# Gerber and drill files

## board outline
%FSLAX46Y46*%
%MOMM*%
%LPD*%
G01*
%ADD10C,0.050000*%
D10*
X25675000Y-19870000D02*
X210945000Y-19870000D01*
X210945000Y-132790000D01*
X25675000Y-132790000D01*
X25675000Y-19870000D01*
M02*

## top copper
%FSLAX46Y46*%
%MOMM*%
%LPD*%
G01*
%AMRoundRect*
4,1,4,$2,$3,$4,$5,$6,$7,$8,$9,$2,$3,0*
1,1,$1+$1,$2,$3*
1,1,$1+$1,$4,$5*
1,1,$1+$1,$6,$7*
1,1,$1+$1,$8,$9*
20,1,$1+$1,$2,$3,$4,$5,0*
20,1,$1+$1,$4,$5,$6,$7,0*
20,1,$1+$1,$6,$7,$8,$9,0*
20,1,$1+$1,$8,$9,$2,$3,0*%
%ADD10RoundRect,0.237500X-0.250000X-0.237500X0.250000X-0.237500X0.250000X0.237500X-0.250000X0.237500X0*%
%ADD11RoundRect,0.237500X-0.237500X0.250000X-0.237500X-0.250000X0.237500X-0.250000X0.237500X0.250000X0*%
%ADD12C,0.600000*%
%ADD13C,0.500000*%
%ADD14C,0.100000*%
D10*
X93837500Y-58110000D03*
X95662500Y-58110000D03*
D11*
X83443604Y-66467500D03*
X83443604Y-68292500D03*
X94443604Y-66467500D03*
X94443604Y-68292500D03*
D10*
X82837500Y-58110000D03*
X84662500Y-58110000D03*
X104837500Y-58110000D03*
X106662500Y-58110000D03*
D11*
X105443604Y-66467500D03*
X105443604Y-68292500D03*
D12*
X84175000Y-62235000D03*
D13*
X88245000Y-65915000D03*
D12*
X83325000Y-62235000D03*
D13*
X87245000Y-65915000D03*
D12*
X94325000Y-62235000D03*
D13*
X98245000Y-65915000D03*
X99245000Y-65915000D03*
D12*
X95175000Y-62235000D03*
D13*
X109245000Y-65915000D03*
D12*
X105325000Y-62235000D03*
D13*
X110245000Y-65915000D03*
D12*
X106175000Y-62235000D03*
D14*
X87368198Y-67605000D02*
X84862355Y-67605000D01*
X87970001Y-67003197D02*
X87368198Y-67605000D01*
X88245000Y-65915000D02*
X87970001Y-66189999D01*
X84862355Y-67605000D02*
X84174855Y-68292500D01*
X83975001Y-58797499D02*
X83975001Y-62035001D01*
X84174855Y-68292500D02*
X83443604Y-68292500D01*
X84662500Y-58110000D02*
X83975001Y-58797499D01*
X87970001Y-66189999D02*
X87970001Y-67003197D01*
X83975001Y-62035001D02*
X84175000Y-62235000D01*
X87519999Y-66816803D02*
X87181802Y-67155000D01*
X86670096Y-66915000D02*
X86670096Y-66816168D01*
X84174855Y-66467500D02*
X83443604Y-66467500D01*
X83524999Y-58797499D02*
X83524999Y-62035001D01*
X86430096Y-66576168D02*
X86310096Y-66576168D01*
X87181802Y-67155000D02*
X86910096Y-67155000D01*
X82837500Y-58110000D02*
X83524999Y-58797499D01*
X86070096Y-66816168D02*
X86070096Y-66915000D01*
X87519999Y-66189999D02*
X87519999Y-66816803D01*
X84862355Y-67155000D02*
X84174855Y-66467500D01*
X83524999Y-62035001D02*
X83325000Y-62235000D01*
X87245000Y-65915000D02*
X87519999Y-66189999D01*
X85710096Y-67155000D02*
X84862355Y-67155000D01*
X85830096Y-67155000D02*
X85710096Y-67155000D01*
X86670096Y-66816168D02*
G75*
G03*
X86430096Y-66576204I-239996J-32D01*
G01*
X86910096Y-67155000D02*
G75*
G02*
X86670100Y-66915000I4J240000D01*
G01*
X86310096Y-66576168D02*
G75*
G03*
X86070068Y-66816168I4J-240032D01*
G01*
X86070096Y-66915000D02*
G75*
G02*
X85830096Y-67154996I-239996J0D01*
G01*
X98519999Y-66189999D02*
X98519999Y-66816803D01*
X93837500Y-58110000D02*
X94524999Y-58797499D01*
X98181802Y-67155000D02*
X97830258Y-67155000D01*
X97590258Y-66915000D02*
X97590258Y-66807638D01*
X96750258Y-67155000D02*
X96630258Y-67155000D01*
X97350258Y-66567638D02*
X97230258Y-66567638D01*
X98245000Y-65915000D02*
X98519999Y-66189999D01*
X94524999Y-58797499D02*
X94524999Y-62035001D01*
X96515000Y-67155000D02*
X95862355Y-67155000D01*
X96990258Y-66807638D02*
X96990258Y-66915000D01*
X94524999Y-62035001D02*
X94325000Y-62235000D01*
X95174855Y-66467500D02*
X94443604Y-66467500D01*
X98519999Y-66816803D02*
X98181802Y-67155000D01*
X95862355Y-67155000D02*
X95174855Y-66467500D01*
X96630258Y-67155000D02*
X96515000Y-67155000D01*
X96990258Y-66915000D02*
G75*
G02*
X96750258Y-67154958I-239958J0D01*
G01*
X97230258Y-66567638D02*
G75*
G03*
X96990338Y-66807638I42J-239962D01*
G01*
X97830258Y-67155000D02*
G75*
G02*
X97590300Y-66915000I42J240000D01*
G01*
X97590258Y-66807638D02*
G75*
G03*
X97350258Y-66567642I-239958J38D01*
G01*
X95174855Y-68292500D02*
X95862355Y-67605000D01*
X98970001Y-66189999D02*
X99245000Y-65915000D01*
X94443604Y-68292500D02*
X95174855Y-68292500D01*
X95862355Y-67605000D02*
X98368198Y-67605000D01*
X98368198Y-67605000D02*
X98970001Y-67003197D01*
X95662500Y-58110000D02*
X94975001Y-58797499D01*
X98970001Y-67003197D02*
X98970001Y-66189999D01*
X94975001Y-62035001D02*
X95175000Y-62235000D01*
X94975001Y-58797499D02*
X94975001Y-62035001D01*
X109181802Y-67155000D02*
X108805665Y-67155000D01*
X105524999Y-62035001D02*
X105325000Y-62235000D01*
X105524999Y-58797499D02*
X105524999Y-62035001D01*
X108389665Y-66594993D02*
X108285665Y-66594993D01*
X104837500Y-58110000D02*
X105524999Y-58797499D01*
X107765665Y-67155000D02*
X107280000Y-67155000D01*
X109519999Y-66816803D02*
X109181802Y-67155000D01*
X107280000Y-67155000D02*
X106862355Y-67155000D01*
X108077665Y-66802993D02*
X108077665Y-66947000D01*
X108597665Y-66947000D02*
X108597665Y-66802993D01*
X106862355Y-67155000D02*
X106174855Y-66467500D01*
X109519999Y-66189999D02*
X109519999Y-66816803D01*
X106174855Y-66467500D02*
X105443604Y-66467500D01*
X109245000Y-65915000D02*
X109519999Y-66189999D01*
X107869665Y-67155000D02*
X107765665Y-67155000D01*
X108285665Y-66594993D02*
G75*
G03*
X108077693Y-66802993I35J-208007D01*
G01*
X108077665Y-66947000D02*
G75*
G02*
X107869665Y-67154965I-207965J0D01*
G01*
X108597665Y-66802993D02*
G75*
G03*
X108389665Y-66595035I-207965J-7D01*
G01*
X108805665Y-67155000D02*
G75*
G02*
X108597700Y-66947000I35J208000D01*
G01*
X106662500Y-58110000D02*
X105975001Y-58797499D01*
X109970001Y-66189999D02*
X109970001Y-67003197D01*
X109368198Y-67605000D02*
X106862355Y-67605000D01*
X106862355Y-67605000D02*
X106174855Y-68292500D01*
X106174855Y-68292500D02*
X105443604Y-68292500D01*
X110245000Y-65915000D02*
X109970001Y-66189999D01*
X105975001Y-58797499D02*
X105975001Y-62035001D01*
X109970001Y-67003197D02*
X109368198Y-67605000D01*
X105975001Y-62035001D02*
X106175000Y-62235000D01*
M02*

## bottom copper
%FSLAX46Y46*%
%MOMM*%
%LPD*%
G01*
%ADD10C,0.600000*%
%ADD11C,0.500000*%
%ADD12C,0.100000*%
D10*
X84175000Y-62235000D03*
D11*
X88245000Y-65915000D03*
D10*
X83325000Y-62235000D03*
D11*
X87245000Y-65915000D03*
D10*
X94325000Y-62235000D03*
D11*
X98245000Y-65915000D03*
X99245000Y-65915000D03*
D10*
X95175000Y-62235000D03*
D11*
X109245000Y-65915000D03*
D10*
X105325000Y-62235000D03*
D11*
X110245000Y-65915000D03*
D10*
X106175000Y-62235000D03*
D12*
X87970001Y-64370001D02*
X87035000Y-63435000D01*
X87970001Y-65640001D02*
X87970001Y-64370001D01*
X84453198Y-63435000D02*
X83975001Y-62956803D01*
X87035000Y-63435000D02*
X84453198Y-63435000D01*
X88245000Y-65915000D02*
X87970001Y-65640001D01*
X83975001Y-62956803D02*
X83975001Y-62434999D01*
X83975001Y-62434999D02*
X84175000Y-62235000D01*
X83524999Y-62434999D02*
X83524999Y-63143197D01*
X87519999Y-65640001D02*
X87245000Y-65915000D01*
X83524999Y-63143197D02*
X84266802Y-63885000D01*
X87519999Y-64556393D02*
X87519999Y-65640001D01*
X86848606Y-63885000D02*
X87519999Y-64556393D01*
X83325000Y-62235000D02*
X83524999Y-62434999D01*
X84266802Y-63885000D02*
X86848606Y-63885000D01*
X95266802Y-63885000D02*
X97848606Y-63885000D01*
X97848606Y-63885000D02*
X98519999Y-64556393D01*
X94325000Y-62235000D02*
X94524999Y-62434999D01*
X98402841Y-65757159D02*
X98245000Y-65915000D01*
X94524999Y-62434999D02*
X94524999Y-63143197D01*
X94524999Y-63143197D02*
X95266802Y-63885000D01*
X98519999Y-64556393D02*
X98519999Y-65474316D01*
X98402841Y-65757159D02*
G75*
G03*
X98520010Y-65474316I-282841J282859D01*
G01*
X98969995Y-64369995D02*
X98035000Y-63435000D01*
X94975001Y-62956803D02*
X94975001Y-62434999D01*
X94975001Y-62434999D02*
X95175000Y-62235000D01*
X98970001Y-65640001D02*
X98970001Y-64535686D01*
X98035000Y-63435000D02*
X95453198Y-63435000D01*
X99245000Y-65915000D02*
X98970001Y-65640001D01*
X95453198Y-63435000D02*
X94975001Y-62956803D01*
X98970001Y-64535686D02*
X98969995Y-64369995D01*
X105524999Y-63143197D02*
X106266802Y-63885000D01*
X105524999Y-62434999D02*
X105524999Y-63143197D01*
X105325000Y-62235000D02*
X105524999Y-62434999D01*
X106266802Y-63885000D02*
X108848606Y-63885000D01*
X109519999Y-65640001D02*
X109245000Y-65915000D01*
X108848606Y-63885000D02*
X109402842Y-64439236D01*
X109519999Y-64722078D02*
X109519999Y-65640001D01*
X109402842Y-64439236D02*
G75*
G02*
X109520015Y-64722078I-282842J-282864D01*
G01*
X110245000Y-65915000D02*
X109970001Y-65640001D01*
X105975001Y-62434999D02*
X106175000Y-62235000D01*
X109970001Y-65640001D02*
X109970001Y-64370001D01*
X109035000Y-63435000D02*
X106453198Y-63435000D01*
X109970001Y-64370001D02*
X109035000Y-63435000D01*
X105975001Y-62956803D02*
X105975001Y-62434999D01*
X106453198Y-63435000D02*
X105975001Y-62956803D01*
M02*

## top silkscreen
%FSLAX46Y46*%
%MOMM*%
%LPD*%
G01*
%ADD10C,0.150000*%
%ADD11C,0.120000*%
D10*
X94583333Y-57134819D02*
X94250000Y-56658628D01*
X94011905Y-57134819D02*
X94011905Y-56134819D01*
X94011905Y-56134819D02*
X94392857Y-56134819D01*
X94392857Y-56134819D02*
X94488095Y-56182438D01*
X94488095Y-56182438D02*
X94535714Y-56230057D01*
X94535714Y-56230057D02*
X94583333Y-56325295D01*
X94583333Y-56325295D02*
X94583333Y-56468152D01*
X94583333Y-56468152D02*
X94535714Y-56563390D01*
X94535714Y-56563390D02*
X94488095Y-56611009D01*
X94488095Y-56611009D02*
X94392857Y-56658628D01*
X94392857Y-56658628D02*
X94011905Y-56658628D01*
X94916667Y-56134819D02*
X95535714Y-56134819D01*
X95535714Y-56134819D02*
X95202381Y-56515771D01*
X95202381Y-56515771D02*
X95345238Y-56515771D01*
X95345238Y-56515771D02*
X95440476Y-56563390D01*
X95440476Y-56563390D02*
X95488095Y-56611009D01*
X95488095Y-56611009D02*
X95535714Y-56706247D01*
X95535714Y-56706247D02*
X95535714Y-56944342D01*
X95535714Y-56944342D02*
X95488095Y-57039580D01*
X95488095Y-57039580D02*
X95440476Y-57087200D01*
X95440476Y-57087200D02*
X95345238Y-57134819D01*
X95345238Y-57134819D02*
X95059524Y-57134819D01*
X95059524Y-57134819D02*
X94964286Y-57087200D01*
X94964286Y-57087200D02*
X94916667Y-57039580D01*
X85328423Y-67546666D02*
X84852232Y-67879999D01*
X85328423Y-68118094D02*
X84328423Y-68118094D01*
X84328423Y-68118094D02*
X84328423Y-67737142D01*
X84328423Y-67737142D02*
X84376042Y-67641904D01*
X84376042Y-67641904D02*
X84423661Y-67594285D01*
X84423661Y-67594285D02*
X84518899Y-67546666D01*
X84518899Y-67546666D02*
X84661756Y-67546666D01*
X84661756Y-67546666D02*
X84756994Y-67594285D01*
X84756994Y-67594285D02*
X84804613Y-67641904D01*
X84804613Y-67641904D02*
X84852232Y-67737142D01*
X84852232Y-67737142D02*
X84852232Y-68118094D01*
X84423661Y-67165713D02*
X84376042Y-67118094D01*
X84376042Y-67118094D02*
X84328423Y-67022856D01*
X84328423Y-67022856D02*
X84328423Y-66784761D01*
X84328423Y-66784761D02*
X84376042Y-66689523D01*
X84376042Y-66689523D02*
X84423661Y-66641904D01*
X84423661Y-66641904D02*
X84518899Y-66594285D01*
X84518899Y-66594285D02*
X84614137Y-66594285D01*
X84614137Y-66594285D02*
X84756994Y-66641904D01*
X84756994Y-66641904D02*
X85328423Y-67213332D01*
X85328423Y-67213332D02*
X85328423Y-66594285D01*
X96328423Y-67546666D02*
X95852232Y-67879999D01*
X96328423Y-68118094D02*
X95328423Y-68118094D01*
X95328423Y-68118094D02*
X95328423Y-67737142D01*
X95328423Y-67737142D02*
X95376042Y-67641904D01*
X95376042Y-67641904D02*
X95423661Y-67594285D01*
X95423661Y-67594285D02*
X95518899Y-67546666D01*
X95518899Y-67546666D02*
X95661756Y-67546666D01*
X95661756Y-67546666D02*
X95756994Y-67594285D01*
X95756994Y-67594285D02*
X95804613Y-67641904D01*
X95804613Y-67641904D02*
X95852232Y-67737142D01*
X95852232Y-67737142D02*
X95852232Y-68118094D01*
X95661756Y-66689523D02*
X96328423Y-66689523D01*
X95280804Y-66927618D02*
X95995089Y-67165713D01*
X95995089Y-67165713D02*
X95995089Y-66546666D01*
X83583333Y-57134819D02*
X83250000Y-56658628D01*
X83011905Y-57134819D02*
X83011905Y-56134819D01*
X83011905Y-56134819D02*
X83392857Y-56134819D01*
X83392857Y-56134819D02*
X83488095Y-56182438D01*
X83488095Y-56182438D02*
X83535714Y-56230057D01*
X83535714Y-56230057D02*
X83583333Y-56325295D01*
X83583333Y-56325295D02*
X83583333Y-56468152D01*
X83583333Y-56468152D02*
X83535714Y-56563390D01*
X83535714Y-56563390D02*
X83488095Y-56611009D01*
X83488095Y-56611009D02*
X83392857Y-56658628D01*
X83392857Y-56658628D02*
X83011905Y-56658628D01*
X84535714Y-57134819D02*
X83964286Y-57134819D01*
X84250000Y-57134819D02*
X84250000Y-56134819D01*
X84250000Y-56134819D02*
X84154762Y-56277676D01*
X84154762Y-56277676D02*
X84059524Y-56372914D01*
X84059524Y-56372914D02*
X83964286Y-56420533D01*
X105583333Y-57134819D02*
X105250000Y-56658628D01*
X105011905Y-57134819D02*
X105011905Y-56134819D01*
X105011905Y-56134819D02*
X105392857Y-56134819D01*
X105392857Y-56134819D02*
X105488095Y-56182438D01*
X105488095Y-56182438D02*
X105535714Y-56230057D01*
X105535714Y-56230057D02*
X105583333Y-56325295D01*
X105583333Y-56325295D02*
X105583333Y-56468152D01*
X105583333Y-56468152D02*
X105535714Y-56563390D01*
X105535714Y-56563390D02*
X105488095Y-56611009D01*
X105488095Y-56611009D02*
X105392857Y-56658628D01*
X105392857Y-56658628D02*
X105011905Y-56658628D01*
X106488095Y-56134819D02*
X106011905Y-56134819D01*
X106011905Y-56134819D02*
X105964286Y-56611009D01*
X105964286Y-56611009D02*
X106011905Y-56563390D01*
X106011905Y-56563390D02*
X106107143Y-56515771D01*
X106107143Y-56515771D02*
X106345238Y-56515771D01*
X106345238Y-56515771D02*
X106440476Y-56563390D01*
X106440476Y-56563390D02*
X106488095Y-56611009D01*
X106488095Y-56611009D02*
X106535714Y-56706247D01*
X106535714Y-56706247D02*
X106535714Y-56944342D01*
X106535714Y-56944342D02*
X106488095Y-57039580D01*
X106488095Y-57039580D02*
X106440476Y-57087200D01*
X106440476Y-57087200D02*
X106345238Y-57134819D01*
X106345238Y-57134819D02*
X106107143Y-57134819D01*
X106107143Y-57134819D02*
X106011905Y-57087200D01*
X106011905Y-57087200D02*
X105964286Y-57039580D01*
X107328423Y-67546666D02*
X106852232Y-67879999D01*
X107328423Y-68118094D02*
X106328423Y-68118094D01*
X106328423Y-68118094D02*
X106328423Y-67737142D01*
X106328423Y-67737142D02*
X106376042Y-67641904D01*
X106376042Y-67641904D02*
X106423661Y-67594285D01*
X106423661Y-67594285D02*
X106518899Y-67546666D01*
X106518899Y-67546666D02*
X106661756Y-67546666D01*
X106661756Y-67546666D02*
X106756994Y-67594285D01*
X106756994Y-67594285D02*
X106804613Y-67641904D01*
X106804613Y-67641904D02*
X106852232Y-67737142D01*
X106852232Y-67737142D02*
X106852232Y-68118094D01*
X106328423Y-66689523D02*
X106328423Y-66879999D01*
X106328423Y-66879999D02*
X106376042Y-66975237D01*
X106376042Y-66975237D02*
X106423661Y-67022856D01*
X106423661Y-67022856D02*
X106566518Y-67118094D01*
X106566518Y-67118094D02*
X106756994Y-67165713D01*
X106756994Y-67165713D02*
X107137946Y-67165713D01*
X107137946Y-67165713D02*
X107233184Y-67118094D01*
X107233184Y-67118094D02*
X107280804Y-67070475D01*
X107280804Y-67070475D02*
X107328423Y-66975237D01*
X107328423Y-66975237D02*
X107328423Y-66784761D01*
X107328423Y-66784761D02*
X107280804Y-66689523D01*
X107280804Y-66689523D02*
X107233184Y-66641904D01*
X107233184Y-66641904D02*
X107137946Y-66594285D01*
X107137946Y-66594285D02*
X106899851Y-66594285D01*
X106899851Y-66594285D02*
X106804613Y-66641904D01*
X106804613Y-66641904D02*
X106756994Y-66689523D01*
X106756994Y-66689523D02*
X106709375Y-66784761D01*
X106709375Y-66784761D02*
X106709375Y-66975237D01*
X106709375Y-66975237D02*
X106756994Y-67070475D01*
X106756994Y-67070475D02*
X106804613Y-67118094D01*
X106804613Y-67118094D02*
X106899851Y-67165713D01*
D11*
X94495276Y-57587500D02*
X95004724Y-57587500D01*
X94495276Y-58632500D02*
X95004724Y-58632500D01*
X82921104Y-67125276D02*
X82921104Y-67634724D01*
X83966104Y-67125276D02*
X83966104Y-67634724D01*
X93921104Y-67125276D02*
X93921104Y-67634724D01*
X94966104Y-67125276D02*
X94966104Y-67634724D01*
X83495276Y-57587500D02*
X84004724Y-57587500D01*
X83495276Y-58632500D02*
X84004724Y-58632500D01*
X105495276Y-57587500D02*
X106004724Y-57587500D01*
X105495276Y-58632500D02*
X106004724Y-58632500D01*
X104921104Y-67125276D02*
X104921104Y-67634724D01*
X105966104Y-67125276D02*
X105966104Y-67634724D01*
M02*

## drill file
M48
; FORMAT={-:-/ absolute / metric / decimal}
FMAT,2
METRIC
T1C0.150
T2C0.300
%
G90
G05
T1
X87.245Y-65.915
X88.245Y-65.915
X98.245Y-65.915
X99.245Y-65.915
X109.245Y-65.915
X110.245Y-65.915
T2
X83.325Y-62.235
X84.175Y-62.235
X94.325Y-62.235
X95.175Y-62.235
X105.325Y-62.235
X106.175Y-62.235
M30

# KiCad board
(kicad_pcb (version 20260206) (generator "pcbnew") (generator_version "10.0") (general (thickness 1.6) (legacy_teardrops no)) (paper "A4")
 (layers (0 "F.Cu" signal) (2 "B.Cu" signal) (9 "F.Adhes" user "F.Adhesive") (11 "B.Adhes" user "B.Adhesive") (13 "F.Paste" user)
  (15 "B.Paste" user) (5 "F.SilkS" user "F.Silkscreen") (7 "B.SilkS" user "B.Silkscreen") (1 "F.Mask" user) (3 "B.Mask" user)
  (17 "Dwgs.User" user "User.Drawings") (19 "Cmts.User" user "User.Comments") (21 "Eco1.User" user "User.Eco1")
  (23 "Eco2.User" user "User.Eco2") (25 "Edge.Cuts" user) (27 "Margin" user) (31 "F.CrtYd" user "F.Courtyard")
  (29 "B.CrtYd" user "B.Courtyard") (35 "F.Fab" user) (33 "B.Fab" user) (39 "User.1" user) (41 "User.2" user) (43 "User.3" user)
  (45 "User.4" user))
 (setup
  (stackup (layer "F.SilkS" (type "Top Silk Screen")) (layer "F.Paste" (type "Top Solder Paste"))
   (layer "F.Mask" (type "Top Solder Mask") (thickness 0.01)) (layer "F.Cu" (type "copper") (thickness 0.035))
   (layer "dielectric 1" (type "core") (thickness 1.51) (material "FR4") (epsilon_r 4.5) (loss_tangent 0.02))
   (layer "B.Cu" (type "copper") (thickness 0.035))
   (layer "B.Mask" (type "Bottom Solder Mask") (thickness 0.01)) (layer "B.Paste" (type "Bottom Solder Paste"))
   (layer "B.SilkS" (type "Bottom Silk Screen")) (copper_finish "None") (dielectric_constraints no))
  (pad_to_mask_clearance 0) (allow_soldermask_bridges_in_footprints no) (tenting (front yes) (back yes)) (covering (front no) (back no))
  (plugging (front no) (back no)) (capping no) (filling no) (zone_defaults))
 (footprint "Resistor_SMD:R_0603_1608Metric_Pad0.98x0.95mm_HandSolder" (layer "F.Cu") (at 94.75 58.11)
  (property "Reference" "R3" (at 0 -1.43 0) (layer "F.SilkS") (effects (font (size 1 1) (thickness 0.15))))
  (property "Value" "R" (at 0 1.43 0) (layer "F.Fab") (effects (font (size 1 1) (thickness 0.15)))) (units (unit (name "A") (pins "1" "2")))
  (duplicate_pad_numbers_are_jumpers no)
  (fp_line (start -0.254724 -0.5225) (end 0.254724 -0.5225) (stroke (width 0.12) (type solid)) (layer "F.SilkS"))
  (fp_line (start -0.254724 0.5225) (end 0.254724 0.5225) (stroke (width 0.12) (type solid)) (layer "F.SilkS"))
  (pad "1" smd roundrect (at -0.9125 0) (size 0.975 0.95) (layers "F.Cu" "F.Mask" "F.Paste") (roundrect_rratio 0.25) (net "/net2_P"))
  (pad "2" smd roundrect (at 0.9125 0) (size 0.975 0.95) (layers "F.Cu" "F.Mask" "F.Paste") (roundrect_rratio 0.25) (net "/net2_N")))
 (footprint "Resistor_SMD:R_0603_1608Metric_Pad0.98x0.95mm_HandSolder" (layer "F.Cu") (at 83.443604 67.38 -90)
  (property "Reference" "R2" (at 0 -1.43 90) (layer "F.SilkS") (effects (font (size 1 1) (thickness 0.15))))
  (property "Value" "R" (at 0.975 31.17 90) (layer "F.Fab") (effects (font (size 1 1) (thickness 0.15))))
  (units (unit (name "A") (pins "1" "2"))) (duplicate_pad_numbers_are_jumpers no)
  (fp_line (start -0.254724 0.5225) (end 0.254724 0.5225) (stroke (width 0.12) (type solid)) (layer "F.SilkS"))
  (fp_line (start -0.254724 -0.5225) (end 0.254724 -0.5225) (stroke (width 0.12) (type solid)) (layer "F.SilkS"))
  (pad "1" smd roundrect (at -0.9125 0 270) (size 0.975 0.95) (layers "F.Cu" "F.Mask" "F.Paste") (roundrect_rratio 0.25) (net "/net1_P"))
  (pad "2" smd roundrect (at 0.9125 0 270) (size 0.975 0.95) (layers "F.Cu" "F.Mask" "F.Paste") (roundrect_rratio 0.25) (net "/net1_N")))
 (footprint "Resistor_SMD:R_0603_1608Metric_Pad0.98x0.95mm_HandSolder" (layer "F.Cu") (at 94.443604 67.38 -90)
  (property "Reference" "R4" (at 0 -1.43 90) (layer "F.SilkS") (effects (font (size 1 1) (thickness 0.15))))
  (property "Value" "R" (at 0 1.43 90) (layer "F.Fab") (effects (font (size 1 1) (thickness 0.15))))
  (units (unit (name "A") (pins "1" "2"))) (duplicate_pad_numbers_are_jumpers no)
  (fp_line (start -0.254724 0.5225) (end 0.254724 0.5225) (stroke (width 0.12) (type solid)) (layer "F.SilkS"))
  (fp_line (start -0.254724 -0.5225) (end 0.254724 -0.5225) (stroke (width 0.12) (type solid)) (layer "F.SilkS"))
  (pad "1" smd roundrect (at -0.9125 0 270) (size 0.975 0.95) (layers "F.Cu" "F.Mask" "F.Paste") (roundrect_rratio 0.25) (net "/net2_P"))
  (pad "2" smd roundrect (at 0.9125 0 270) (size 0.975 0.95) (layers "F.Cu" "F.Mask" "F.Paste") (roundrect_rratio 0.25) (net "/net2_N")))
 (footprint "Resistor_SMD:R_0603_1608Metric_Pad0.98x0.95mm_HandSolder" (layer "F.Cu") (at 83.75 58.11)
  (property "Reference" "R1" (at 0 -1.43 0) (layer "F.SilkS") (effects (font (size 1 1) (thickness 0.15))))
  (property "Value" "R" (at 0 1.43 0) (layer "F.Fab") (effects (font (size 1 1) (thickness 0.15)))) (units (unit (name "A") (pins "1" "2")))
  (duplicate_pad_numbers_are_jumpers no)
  (fp_line (start -0.254724 -0.5225) (end 0.254724 -0.5225) (stroke (width 0.12) (type solid)) (layer "F.SilkS"))
  (fp_line (start -0.254724 0.5225) (end 0.254724 0.5225) (stroke (width 0.12) (type solid)) (layer "F.SilkS"))
  (pad "1" smd roundrect (at -0.9125 0) (size 0.975 0.95) (layers "F.Cu" "F.Mask" "F.Paste") (roundrect_rratio 0.25) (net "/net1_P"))
  (pad "2" smd roundrect (at 0.9125 0) (size 0.975 0.95) (layers "F.Cu" "F.Mask" "F.Paste") (roundrect_rratio 0.25) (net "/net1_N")))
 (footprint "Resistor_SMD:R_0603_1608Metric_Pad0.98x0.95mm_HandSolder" (layer "F.Cu") (at 105.75 58.11)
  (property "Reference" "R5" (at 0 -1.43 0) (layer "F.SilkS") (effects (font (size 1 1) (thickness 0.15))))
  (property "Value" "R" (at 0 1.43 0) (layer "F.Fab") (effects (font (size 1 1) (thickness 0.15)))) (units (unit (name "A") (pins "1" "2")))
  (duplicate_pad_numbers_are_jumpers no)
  (fp_line (start -0.254724 -0.5225) (end 0.254724 -0.5225) (stroke (width 0.12) (type solid)) (layer "F.SilkS"))
  (fp_line (start -0.254724 0.5225) (end 0.254724 0.5225) (stroke (width 0.12) (type solid)) (layer "F.SilkS"))
  (pad "1" smd roundrect (at -0.9125 0) (size 0.975 0.95) (layers "F.Cu" "F.Mask" "F.Paste") (roundrect_rratio 0.25) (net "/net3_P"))
  (pad "2" smd roundrect (at 0.9125 0) (size 0.975 0.95) (layers "F.Cu" "F.Mask" "F.Paste") (roundrect_rratio 0.25) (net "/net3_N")))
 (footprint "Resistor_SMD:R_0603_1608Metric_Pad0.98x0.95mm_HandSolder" (layer "F.Cu") (at 105.443604 67.38 -90)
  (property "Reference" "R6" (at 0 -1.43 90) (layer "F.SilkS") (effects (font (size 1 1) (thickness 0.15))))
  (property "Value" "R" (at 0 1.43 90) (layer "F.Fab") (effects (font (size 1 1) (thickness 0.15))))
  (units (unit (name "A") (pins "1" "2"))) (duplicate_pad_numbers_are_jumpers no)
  (fp_line (start -0.254724 0.5225) (end 0.254724 0.5225) (stroke (width 0.12) (type solid)) (layer "F.SilkS"))
  (fp_line (start -0.254724 -0.5225) (end 0.254724 -0.5225) (stroke (width 0.12) (type solid)) (layer "F.SilkS"))
  (pad "1" smd roundrect (at -0.9125 0 270) (size 0.975 0.95) (layers "F.Cu" "F.Mask" "F.Paste") (roundrect_rratio 0.25) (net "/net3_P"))
  (pad "2" smd roundrect (at 0.9125 0 270) (size 0.975 0.95) (layers "F.Cu" "F.Mask" "F.Paste") (roundrect_rratio 0.25) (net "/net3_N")))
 (gr_rect (start 25.675 19.87) (end 210.945 132.79) (stroke (width 0.05) (type default)) (fill no) (layer "Edge.Cuts"))
 (segment (start 87.368198 67.605) (end 84.862355 67.605) (width 0.1) (layer "F.Cu") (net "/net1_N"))
 (segment (start 87.970001 67.003197) (end 87.368198 67.605) (width 0.1) (layer "F.Cu") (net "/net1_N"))
 (segment (start 88.245 65.915) (end 87.970001 66.189999) (width 0.1) (layer "F.Cu") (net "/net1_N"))
 (segment (start 84.862355 67.605) (end 84.174855 68.2925) (width 0.1) (layer "F.Cu") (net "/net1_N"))
 (segment (start 83.975001 58.797499) (end 83.975001 62.035001) (width 0.1) (layer "F.Cu") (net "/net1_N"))
 (segment (start 84.174855 68.2925) (end 83.443604 68.2925) (width 0.1) (layer "F.Cu") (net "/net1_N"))
 (segment (start 84.6625 58.11) (end 83.975001 58.797499) (width 0.1) (layer "F.Cu") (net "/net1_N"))
 (segment (start 87.970001 66.189999) (end 87.970001 67.003197) (width 0.1) (layer "F.Cu") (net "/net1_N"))
 (segment (start 83.975001 62.035001) (end 84.175 62.235) (width 0.1) (layer "F.Cu") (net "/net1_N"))
 (via (at 84.175 62.235) (size 0.6) (drill 0.3) (layers "F.Cu" "B.Cu") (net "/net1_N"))
 (via (at 88.245 65.915) (size 0.5) (drill 0.15) (layers "F.Cu" "B.Cu") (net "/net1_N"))
 (segment (start 87.970001 64.370001) (end 87.035 63.435) (width 0.1) (layer "B.Cu") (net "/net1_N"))
 (segment (start 87.970001 65.640001) (end 87.970001 64.370001) (width 0.1) (layer "B.Cu") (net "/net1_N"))
 (segment (start 84.453198 63.435) (end 83.975001 62.956803) (width 0.1) (layer "B.Cu") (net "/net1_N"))
 (segment (start 87.035 63.435) (end 84.453198 63.435) (width 0.1) (layer "B.Cu") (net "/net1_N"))
 (segment (start 88.245 65.915) (end 87.970001 65.640001) (width 0.1) (layer "B.Cu") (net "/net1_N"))
 (segment (start 83.975001 62.956803) (end 83.975001 62.434999) (width 0.1) (layer "B.Cu") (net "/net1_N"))
 (segment (start 83.975001 62.434999) (end 84.175 62.235) (width 0.1) (layer "B.Cu") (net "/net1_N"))
 (segment (start 87.519999 66.816803) (end 87.181802 67.155) (width 0.1) (layer "F.Cu") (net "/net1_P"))
 (segment (start 86.670096 66.915) (end 86.670096 66.816168) (width 0.1) (layer "F.Cu") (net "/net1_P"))
 (segment (start 84.174855 66.4675) (end 83.443604 66.4675) (width 0.1) (layer "F.Cu") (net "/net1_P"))
 (segment (start 83.524999 58.797499) (end 83.524999 62.035001) (width 0.1) (layer "F.Cu") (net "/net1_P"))
 (segment (start 86.430096 66.576168) (end 86.310096 66.576168) (width 0.1) (layer "F.Cu") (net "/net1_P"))
 (segment (start 87.181802 67.155) (end 86.910096 67.155) (width 0.1) (layer "F.Cu") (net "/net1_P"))
 (segment (start 82.8375 58.11) (end 83.524999 58.797499) (width 0.1) (layer "F.Cu") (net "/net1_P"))
 (segment (start 86.070096 66.816168) (end 86.070096 66.915) (width 0.1) (layer "F.Cu") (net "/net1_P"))
 (segment (start 87.519999 66.189999) (end 87.519999 66.816803) (width 0.1) (layer "F.Cu") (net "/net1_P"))
 (segment (start 84.862355 67.155) (end 84.174855 66.4675) (width 0.1) (layer "F.Cu") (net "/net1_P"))
 (segment (start 83.524999 62.035001) (end 83.325 62.235) (width 0.1) (layer "F.Cu") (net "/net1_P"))
 (segment (start 87.245 65.915) (end 87.519999 66.189999) (width 0.1) (layer "F.Cu") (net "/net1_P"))
 (segment (start 85.710096 67.155) (end 84.862355 67.155) (width 0.1) (layer "F.Cu") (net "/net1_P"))
 (segment (start 85.830096 67.155) (end 85.710096 67.155) (width 0.1) (layer "F.Cu") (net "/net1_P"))
 (via (at 83.325 62.235) (size 0.6) (drill 0.3) (layers "F.Cu" "B.Cu") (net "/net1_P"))
 (via (at 87.245 65.915) (size 0.5) (drill 0.15) (layers "F.Cu" "B.Cu") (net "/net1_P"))
 (arc (start 86.670096 66.816168) (mid 86.599802 66.646462) (end 86.430096 66.576168) (width 0.1) (layer "F.Cu") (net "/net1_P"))
 (arc (start 86.910096 67.155) (mid 86.74039 67.084706) (end 86.670096 66.915) (width 0.1) (layer "F.Cu") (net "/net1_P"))
 (arc (start 86.310096 66.576168) (mid 86.14039 66.646462) (end 86.070096 66.816168) (width 0.1) (layer "F.Cu") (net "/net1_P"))
 (arc (start 86.070096 66.915) (mid 85.999802 67.084706) (end 85.830096 67.155) (width 0.1) (layer "F.Cu") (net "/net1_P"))
 (segment (start 83.524999 62.434999) (end 83.524999 63.143197) (width 0.1) (layer "B.Cu") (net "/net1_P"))
 (segment (start 87.519999 65.640001) (end 87.245 65.915) (width 0.1) (layer "B.Cu") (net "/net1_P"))
 (segment (start 83.524999 63.143197) (end 84.266802 63.885) (width 0.1) (layer "B.Cu") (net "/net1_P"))
 (segment (start 87.519999 64.556393) (end 87.519999 65.640001) (width 0.1) (layer "B.Cu") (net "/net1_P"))
 (segment (start 86.848606 63.885) (end 87.519999 64.556393) (width 0.1) (layer "B.Cu") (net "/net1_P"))
 (segment (start 83.325 62.235) (end 83.524999 62.434999) (width 0.1) (layer "B.Cu") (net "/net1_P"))
 (segment (start 84.266802 63.885) (end 86.848606 63.885) (width 0.1) (layer "B.Cu") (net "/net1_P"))
 (segment (start 98.519999 66.189999) (end 98.519999 66.816803) (width 0.1) (layer "F.Cu") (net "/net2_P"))
 (segment (start 93.8375 58.11) (end 94.524999 58.797499) (width 0.1) (layer "F.Cu") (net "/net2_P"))
 (segment (start 98.181802 67.155) (end 97.830258 67.155) (width 0.1) (layer "F.Cu") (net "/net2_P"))
 (segment (start 97.590258 66.915) (end 97.590258 66.807638) (width 0.1) (layer "F.Cu") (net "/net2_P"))
 (segment (start 96.750258 67.155) (end 96.630258 67.155) (width 0.1) (layer "F.Cu") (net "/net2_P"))
 (segment (start 97.350258 66.567638) (end 97.230258 66.567638) (width 0.1) (layer "F.Cu") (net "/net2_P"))
 (segment (start 98.245 65.915) (end 98.519999 66.189999) (width 0.1) (layer "F.Cu") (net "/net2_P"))
 (segment (start 94.524999 58.797499) (end 94.524999 62.035001) (width 0.1) (layer "F.Cu") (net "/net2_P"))
 (segment (start 96.515 67.155) (end 95.862355 67.155) (width 0.1) (layer "F.Cu") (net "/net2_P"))
 (segment (start 96.990258 66.807638) (end 96.990258 66.915) (width 0.1) (layer "F.Cu") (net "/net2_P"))
 (segment (start 94.524999 62.035001) (end 94.325 62.235) (width 0.1) (layer "F.Cu") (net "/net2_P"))
 (segment (start 95.174855 66.4675) (end 94.443604 66.4675) (width 0.1) (layer "F.Cu") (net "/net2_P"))
 (segment (start 98.519999 66.816803) (end 98.181802 67.155) (width 0.1) (layer "F.Cu") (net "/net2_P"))
 (segment (start 95.862355 67.155) (end 95.174855 66.4675) (width 0.1) (layer "F.Cu") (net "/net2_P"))
 (segment (start 96.630258 67.155) (end 96.515 67.155) (width 0.1) (layer "F.Cu") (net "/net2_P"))
 (via (at 94.325 62.235) (size 0.6) (drill 0.3) (layers "F.Cu" "B.Cu") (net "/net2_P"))
 (via (at 98.245 65.915) (size 0.5) (drill 0.15) (layers "F.Cu" "B.Cu") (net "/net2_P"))
 (arc (start 96.990258 66.915) (mid 96.919964 67.084706) (end 96.750258 67.155) (width 0.1) (layer "F.Cu") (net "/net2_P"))
 (arc (start 97.230258 66.567638) (mid 97.060552 66.637932) (end 96.990258 66.807638) (width 0.1) (layer "F.Cu") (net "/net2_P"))
 (arc (start 97.830258 67.155) (mid 97.660552 67.084706) (end 97.590258 66.915) (width 0.1) (layer "F.Cu") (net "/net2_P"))
 (arc (start 97.590258 66.807638) (mid 97.519964 66.637932) (end 97.350258 66.567638) (width 0.1) (layer "F.Cu") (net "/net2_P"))
 (segment (start 95.266802 63.885) (end 97.848606 63.885) (width 0.1) (layer "B.Cu") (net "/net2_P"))
 (segment (start 97.848606 63.885) (end 98.519999 64.556393) (width 0.1) (layer "B.Cu") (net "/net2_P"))
 (segment (start 94.325 62.235) (end 94.524999 62.434999) (width 0.1) (layer "B.Cu") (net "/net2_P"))
 (segment (start 98.402841 65.757159) (end 98.245 65.915) (width 0.1) (layer "B.Cu") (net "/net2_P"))
 (segment (start 94.524999 62.434999) (end 94.524999 63.143197) (width 0.1) (layer "B.Cu") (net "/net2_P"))
 (segment (start 94.524999 63.143197) (end 95.266802 63.885) (width 0.1) (layer "B.Cu") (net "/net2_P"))
 (segment (start 98.519999 64.556393) (end 98.519999 65.474316) (width 0.1) (layer "B.Cu") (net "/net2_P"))
 (arc (start 98.402841 65.757159) (mid 98.48955 65.62739) (end 98.519999 65.474316) (width 0.1) (layer "B.Cu") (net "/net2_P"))
 (segment (start 95.174855 68.2925) (end 95.862355 67.605) (width 0.1) (layer "F.Cu") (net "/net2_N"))
 (segment (start 98.970001 66.189999) (end 99.245 65.915) (width 0.1) (layer "F.Cu") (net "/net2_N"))
 (segment (start 94.443604 68.2925) (end 95.174855 68.2925) (width 0.1) (layer "F.Cu") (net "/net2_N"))
 (segment (start 95.862355 67.605) (end 98.368198 67.605) (width 0.1) (layer "F.Cu") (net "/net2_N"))
 (segment (start 98.368198 67.605) (end 98.970001 67.003197) (width 0.1) (layer "F.Cu") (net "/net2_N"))
 (segment (start 95.6625 58.11) (end 94.975001 58.797499) (width 0.1) (layer "F.Cu") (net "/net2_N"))
 (segment (start 98.970001 67.003197) (end 98.970001 66.189999) (width 0.1) (layer "F.Cu") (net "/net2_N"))
 (segment (start 94.975001 62.035001) (end 95.175 62.235) (width 0.1) (layer "F.Cu") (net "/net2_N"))
 (segment (start 94.975001 58.797499) (end 94.975001 62.035001) (width 0.1) (layer "F.Cu") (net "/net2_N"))
 (via (at 99.245 65.915) (size 0.5) (drill 0.15) (layers "F.Cu" "B.Cu") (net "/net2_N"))
 (via (at 95.175 62.235) (size 0.6) (drill 0.3) (layers "F.Cu" "B.Cu") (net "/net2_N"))
 (segment (start 98.969995 64.369995) (end 98.035 63.435) (width 0.1) (layer "B.Cu") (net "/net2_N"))
 (segment (start 94.975001 62.956803) (end 94.975001 62.434999) (width 0.1) (layer "B.Cu") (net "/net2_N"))
 (segment (start 94.975001 62.434999) (end 95.175 62.235) (width 0.1) (layer "B.Cu") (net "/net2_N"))
 (segment (start 98.970001 65.640001) (end 98.970001 64.535686) (width 0.1) (layer "B.Cu") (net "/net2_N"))
 (segment (start 98.035 63.435) (end 95.453198 63.435) (width 0.1) (layer "B.Cu") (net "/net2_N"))
 (segment (start 99.245 65.915) (end 98.970001 65.640001) (width 0.1) (layer "B.Cu") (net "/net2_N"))
 (segment (start 95.453198 63.435) (end 94.975001 62.956803) (width 0.1) (layer "B.Cu") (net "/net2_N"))
 (segment (start 98.970001 64.535686) (end 98.969995 64.369995) (width 0.1) (layer "B.Cu") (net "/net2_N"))
 (segment (start 109.181802 67.155) (end 108.805665 67.155) (width 0.1) (layer "F.Cu") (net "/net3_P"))
 (segment (start 105.524999 62.035001) (end 105.325 62.235) (width 0.1) (layer "F.Cu") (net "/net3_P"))
 (segment (start 105.524999 58.797499) (end 105.524999 62.035001) (width 0.1) (layer "F.Cu") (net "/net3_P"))
 (segment (start 108.389665 66.594993) (end 108.285665 66.594993) (width 0.1) (layer "F.Cu") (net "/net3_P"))
 (segment (start 104.8375 58.11) (end 105.524999 58.797499) (width 0.1) (layer "F.Cu") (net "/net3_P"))
 (segment (start 107.765665 67.155) (end 107.28 67.155) (width 0.1) (layer "F.Cu") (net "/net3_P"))
 (segment (start 109.519999 66.816803) (end 109.181802 67.155) (width 0.1) (layer "F.Cu") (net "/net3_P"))
 (segment (start 107.28 67.155) (end 106.862355 67.155) (width 0.1) (layer "F.Cu") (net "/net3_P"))
 (segment (start 108.077665 66.802993) (end 108.077665 66.947) (width 0.1) (layer "F.Cu") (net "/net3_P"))
 (segment (start 108.597665 66.947) (end 108.597665 66.802993) (width 0.1) (layer "F.Cu") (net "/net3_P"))
 (segment (start 106.862355 67.155) (end 106.174855 66.4675) (width 0.1) (layer "F.Cu") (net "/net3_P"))
 (segment (start 109.519999 66.189999) (end 109.519999 66.816803) (width 0.1) (layer "F.Cu") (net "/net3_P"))
 (segment (start 106.174855 66.4675) (end 105.443604 66.4675) (width 0.1) (layer "F.Cu") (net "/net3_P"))
 (segment (start 109.245 65.915) (end 109.519999 66.189999) (width 0.1) (layer "F.Cu") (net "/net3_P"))
 (segment (start 107.869665 67.155) (end 107.765665 67.155) (width 0.1) (layer "F.Cu") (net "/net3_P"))
 (via (at 109.245 65.915) (size 0.5) (drill 0.15) (layers "F.Cu" "B.Cu") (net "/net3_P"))
 (via (at 105.325 62.235) (size 0.6) (drill 0.3) (layers "F.Cu" "B.Cu") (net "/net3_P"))
 (arc (start 108.285665 66.594993) (mid 108.138587 66.655915) (end 108.077665 66.802993) (width 0.1) (layer "F.Cu") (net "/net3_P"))
 (arc (start 108.077665 66.947) (mid 108.016743 67.094078) (end 107.869665 67.155) (width 0.1) (layer "F.Cu") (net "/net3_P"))
 (arc (start 108.597665 66.802993) (mid 108.536743 66.655915) (end 108.389665 66.594993) (width 0.1) (layer "F.Cu") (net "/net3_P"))
 (arc (start 108.805665 67.155) (mid 108.658587 67.094078) (end 108.597665 66.947) (width 0.1) (layer "F.Cu") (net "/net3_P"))
 (segment (start 105.524999 63.143197) (end 106.266802 63.885) (width 0.1) (layer "B.Cu") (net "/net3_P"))
 (segment (start 105.524999 62.434999) (end 105.524999 63.143197) (width 0.1) (layer "B.Cu") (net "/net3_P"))
 (segment (start 105.325 62.235) (end 105.524999 62.434999) (width 0.1) (layer "B.Cu") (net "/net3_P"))
 (segment (start 106.266802 63.885) (end 108.848606 63.885) (width 0.1) (layer "B.Cu") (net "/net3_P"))
 (segment (start 109.519999 65.640001) (end 109.245 65.915) (width 0.1) (layer "B.Cu") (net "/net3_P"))
 (segment (start 108.848606 63.885) (end 109.402842 64.439236) (width 0.1) (layer "B.Cu") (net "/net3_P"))
 (segment (start 109.519999 64.722078) (end 109.519999 65.640001) (width 0.1) (layer "B.Cu") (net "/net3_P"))
 (arc (start 109.402842 64.439236) (mid 109.489551 64.569005) (end 109.519999 64.722078) (width 0.1) (layer "B.Cu") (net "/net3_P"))
 (segment (start 106.6625 58.11) (end 105.975001 58.797499) (width 0.1) (layer "F.Cu") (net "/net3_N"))
 (segment (start 109.970001 66.189999) (end 109.970001 67.003197) (width 0.1) (layer "F.Cu") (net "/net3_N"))
 (segment (start 109.368198 67.605) (end 106.862355 67.605) (width 0.1) (layer "F.Cu") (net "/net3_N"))
 (segment (start 106.862355 67.605) (end 106.174855 68.2925) (width 0.1) (layer "F.Cu") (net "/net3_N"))
 (segment (start 106.174855 68.2925) (end 105.443604 68.2925) (width 0.1) (layer "F.Cu") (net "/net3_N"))
 (segment (start 110.245 65.915) (end 109.970001 66.189999) (width 0.1) (layer "F.Cu") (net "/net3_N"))
 (segment (start 105.975001 58.797499) (end 105.975001 62.035001) (width 0.1) (layer "F.Cu") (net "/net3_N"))
 (segment (start 109.970001 67.003197) (end 109.368198 67.605) (width 0.1) (layer "F.Cu") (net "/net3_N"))
 (segment (start 105.975001 62.035001) (end 106.175 62.235) (width 0.1) (layer "F.Cu") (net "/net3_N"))
 (via (at 110.245 65.915) (size 0.5) (drill 0.15) (layers "F.Cu" "B.Cu") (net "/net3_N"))
 (via (at 106.175 62.235) (size 0.6) (drill 0.3) (layers "F.Cu" "B.Cu") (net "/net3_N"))
 (segment (start 110.245 65.915) (end 109.970001 65.640001) (width 0.1) (layer "B.Cu") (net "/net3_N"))
 (segment (start 105.975001 62.434999) (end 106.175 62.235) (width 0.1) (layer "B.Cu") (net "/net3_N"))
 (segment (start 109.970001 65.640001) (end 109.970001 64.370001) (width 0.1) (layer "B.Cu") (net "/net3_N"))
 (segment (start 109.035 63.435) (end 106.453198 63.435) (width 0.1) (layer "B.Cu") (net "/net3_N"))
 (segment (start 109.970001 64.370001) (end 109.035 63.435) (width 0.1) (layer "B.Cu") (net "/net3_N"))
 (segment (start 105.975001 62.956803) (end 105.975001 62.434999) (width 0.1) (layer "B.Cu") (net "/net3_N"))
 (segment (start 106.453198 63.435) (end 105.975001 62.956803) (width 0.1) (layer "B.Cu") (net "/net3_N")))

